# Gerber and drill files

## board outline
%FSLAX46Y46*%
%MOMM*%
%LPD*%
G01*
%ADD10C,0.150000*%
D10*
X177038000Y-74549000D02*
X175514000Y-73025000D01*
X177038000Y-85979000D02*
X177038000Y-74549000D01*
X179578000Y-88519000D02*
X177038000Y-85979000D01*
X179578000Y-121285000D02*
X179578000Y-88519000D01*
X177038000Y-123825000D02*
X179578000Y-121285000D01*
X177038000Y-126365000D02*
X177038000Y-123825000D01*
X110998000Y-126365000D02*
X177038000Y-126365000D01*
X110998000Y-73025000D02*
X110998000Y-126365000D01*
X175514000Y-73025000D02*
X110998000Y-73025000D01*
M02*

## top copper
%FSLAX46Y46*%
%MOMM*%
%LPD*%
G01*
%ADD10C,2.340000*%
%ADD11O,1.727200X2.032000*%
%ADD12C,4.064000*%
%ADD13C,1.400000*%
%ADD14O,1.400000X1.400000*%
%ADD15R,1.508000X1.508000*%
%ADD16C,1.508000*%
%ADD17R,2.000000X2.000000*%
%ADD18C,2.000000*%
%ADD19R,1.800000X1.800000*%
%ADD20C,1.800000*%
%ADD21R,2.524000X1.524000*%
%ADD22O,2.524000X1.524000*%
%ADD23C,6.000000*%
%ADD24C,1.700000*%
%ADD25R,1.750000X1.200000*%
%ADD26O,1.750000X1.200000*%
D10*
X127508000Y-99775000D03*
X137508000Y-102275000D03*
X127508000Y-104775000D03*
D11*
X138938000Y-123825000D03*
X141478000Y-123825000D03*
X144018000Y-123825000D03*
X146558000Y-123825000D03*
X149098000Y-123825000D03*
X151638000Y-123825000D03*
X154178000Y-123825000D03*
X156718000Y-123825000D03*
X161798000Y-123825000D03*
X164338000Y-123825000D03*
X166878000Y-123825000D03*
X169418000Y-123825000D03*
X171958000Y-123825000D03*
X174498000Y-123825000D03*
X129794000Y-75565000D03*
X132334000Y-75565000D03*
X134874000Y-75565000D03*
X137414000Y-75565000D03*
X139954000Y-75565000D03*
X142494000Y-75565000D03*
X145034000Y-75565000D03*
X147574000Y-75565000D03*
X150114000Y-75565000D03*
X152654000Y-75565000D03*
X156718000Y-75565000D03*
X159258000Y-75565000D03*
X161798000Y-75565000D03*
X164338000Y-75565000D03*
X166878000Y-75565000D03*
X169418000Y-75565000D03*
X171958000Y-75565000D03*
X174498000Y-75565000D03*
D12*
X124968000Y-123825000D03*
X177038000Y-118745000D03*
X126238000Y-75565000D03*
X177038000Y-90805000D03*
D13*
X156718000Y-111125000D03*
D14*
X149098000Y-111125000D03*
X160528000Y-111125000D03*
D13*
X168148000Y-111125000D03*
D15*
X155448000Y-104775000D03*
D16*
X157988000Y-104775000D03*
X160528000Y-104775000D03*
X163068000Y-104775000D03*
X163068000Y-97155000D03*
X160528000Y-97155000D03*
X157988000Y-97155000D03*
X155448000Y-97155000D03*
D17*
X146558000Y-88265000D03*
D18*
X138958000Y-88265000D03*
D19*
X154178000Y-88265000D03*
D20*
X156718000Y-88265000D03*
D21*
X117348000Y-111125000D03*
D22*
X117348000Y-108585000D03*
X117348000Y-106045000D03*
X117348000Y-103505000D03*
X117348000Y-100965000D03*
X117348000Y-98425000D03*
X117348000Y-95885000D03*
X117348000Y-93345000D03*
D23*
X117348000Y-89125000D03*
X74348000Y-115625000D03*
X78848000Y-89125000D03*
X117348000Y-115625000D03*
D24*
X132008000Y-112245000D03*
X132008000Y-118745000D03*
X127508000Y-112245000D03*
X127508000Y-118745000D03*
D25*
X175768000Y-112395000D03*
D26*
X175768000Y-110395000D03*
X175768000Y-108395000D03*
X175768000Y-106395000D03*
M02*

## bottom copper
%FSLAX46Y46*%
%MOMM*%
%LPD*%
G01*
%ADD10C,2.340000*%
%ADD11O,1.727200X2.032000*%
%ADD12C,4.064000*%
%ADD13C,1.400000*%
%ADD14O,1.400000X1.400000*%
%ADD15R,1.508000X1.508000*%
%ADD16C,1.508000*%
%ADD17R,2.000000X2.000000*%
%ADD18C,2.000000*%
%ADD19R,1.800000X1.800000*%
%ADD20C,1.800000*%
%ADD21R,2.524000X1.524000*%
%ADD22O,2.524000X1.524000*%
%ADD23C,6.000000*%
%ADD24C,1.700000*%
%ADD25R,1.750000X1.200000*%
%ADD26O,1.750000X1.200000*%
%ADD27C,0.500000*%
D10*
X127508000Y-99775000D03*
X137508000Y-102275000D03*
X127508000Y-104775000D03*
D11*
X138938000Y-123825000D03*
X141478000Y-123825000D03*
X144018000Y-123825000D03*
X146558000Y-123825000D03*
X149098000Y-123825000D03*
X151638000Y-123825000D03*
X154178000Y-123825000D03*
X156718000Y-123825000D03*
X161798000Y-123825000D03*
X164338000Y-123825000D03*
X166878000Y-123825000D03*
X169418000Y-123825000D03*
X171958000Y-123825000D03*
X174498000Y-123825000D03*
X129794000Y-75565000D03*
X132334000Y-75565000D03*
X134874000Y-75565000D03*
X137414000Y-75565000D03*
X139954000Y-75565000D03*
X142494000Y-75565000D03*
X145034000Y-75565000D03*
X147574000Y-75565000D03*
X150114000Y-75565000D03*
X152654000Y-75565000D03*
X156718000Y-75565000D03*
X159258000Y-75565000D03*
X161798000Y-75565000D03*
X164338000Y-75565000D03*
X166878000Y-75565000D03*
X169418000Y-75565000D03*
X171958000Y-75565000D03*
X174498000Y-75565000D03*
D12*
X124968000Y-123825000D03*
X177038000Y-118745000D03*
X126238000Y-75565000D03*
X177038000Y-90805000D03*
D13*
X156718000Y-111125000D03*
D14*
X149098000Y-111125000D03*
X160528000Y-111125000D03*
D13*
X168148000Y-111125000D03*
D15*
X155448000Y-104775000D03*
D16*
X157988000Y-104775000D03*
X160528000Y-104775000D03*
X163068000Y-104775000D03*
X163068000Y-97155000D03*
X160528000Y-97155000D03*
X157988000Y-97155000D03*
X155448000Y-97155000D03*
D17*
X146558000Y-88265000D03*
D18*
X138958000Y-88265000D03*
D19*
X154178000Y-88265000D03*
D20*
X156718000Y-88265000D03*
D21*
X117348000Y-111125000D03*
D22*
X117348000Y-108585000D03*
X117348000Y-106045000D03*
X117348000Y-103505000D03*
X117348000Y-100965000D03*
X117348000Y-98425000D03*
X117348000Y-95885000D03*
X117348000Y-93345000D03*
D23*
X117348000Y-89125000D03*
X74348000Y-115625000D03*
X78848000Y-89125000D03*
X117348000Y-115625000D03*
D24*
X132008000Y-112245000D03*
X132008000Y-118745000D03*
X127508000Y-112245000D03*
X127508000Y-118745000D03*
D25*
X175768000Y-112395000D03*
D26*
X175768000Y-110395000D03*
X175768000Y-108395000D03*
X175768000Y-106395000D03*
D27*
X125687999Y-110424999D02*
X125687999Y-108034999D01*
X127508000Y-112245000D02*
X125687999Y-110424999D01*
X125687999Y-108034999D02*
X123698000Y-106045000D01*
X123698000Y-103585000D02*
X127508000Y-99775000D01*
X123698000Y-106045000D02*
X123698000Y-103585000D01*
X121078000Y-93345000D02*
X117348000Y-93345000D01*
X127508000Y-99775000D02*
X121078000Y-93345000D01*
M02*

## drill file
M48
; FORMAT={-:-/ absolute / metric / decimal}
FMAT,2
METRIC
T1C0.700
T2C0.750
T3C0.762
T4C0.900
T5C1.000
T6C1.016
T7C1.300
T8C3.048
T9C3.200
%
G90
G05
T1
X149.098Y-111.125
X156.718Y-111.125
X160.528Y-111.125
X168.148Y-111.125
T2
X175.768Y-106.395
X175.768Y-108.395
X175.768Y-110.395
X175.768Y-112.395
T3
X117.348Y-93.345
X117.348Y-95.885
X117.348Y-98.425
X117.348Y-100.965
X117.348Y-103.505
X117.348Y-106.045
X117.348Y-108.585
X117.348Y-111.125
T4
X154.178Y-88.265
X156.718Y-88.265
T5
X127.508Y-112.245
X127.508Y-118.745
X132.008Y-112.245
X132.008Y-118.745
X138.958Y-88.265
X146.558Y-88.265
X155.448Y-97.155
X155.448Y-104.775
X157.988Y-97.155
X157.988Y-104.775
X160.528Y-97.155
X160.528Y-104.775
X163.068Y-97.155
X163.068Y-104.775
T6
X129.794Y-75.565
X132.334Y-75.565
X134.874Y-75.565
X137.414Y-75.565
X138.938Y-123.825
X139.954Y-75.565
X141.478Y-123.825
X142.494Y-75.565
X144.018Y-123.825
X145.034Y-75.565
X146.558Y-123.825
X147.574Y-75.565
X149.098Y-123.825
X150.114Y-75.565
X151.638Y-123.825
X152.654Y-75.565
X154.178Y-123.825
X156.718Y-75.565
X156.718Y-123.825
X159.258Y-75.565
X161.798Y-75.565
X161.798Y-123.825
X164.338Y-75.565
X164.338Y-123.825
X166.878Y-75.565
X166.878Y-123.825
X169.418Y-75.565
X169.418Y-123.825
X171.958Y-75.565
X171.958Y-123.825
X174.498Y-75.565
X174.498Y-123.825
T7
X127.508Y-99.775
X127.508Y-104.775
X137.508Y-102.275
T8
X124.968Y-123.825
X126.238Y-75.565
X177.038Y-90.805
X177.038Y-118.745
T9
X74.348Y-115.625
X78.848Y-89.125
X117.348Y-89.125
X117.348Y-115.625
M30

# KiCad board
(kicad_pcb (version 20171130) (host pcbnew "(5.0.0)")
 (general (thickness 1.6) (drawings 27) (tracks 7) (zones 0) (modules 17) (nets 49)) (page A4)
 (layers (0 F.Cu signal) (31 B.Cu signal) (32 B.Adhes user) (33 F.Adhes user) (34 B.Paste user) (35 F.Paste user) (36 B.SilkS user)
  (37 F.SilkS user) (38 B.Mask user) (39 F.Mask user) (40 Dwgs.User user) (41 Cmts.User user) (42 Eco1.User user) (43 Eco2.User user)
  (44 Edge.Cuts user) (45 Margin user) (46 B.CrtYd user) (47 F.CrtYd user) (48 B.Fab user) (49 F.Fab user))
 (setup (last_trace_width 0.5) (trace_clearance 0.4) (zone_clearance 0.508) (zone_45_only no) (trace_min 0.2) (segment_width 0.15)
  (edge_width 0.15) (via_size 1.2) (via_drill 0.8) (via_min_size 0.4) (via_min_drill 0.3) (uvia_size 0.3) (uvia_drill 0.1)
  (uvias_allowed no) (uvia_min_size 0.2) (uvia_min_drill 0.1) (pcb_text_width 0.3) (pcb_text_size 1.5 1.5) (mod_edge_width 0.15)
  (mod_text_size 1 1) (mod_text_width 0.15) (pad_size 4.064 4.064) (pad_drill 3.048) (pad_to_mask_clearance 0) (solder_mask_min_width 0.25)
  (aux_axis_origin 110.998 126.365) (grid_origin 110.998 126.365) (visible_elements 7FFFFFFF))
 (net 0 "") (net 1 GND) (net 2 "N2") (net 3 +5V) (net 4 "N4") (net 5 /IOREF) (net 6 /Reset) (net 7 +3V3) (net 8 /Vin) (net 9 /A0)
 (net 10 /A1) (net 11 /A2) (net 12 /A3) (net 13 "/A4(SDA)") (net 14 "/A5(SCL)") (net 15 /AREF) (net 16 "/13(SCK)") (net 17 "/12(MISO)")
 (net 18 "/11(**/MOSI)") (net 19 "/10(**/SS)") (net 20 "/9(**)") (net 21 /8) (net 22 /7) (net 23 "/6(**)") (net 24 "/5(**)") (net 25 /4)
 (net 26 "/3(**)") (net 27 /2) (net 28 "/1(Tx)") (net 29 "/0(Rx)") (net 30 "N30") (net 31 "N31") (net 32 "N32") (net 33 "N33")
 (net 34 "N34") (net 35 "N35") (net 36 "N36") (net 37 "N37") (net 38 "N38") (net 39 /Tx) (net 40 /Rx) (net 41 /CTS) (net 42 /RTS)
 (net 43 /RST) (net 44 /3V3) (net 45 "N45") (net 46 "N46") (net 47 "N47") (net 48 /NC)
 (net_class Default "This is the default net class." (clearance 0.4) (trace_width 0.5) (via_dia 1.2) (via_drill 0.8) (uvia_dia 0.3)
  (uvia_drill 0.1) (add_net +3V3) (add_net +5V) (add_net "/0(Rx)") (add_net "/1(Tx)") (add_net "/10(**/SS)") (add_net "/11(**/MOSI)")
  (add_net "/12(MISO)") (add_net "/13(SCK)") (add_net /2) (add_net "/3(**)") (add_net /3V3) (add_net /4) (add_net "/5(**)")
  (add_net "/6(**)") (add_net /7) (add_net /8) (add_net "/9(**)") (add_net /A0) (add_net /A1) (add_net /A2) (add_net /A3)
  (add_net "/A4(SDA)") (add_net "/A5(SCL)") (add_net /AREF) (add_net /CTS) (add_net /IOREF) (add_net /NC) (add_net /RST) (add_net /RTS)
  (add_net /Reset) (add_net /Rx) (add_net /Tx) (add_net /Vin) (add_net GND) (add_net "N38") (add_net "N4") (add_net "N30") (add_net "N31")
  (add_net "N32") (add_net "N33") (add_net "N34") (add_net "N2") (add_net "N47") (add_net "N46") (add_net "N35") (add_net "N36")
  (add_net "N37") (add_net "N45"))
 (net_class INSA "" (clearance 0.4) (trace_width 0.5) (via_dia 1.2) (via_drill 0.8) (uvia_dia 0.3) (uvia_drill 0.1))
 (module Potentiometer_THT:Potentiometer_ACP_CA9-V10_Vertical (layer F.Cu) (at 127.508 104.775)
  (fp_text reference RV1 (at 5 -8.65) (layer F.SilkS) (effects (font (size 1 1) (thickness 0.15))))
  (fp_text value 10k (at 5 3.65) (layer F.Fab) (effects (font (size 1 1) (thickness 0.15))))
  (pad 3 thru_hole circle (at 0 -5) (size 2.34 2.34) (drill 1.3) (layers *.Cu *.Mask) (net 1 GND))
  (pad 2 thru_hole circle (at 10 -2.5) (size 2.34 2.34) (drill 1.3) (layers *.Cu *.Mask) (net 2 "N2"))
  (pad 1 thru_hole circle (at 0 0) (size 2.34 2.34) (drill 1.3) (layers *.Cu *.Mask) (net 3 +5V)))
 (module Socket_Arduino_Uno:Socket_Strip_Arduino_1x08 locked (layer F.Cu) (at 138.938 123.825)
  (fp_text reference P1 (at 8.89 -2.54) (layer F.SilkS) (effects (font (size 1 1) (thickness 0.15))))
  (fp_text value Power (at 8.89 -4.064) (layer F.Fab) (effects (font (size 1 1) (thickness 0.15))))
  (pad 1 thru_hole oval (at 0 0) (size 1.7272 2.032) (drill 1.016) (layers *.Cu *.Mask F.SilkS) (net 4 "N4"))
  (pad 2 thru_hole oval (at 2.54 0) (size 1.7272 2.032) (drill 1.016) (layers *.Cu *.Mask F.SilkS) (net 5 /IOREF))
  (pad 3 thru_hole oval (at 5.08 0) (size 1.7272 2.032) (drill 1.016) (layers *.Cu *.Mask F.SilkS) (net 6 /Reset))
  (pad 4 thru_hole oval (at 7.62 0) (size 1.7272 2.032) (drill 1.016) (layers *.Cu *.Mask F.SilkS) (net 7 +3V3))
  (pad 5 thru_hole oval (at 10.16 0) (size 1.7272 2.032) (drill 1.016) (layers *.Cu *.Mask F.SilkS) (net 3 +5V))
  (pad 6 thru_hole oval (at 12.7 0) (size 1.7272 2.032) (drill 1.016) (layers *.Cu *.Mask F.SilkS) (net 1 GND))
  (pad 7 thru_hole oval (at 15.24 0) (size 1.7272 2.032) (drill 1.016) (layers *.Cu *.Mask F.SilkS) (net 1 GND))
  (pad 8 thru_hole oval (at 17.78 0) (size 1.7272 2.032) (drill 1.016) (layers *.Cu *.Mask F.SilkS) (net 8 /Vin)))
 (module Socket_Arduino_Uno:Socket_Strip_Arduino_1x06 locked (layer F.Cu) (at 161.798 123.825)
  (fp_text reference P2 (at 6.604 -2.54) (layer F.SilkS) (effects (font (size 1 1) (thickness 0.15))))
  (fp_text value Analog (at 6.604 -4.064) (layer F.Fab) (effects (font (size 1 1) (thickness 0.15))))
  (pad 1 thru_hole oval (at 0 0) (size 1.7272 2.032) (drill 1.016) (layers *.Cu *.Mask F.SilkS) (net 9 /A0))
  (pad 2 thru_hole oval (at 2.54 0) (size 1.7272 2.032) (drill 1.016) (layers *.Cu *.Mask F.SilkS) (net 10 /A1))
  (pad 3 thru_hole oval (at 5.08 0) (size 1.7272 2.032) (drill 1.016) (layers *.Cu *.Mask F.SilkS) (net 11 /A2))
  (pad 4 thru_hole oval (at 7.62 0) (size 1.7272 2.032) (drill 1.016) (layers *.Cu *.Mask F.SilkS) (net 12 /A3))
  (pad 5 thru_hole oval (at 10.16 0) (size 1.7272 2.032) (drill 1.016) (layers *.Cu *.Mask F.SilkS) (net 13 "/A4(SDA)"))
  (pad 6 thru_hole oval (at 12.7 0) (size 1.7272 2.032) (drill 1.016) (layers *.Cu *.Mask F.SilkS) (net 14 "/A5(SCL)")))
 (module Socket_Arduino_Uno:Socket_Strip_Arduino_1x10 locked (layer F.Cu) (at 129.794 75.565)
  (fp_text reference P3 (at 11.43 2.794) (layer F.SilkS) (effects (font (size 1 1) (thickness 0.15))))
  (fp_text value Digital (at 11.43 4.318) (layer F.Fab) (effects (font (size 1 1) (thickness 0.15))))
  (pad 1 thru_hole oval (at 0 0) (size 1.7272 2.032) (drill 1.016) (layers *.Cu *.Mask F.SilkS) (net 14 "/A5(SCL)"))
  (pad 2 thru_hole oval (at 2.54 0) (size 1.7272 2.032) (drill 1.016) (layers *.Cu *.Mask F.SilkS) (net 13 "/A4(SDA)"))
  (pad 3 thru_hole oval (at 5.08 0) (size 1.7272 2.032) (drill 1.016) (layers *.Cu *.Mask F.SilkS) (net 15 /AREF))
  (pad 4 thru_hole oval (at 7.62 0) (size 1.7272 2.032) (drill 1.016) (layers *.Cu *.Mask F.SilkS) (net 1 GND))
  (pad 5 thru_hole oval (at 10.16 0) (size 1.7272 2.032) (drill 1.016) (layers *.Cu *.Mask F.SilkS) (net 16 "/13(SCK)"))
  (pad 6 thru_hole oval (at 12.7 0) (size 1.7272 2.032) (drill 1.016) (layers *.Cu *.Mask F.SilkS) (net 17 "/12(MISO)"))
  (pad 7 thru_hole oval (at 15.24 0) (size 1.7272 2.032) (drill 1.016) (layers *.Cu *.Mask F.SilkS) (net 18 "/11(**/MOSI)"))
  (pad 8 thru_hole oval (at 17.78 0) (size 1.7272 2.032) (drill 1.016) (layers *.Cu *.Mask F.SilkS) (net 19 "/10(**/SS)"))
  (pad 9 thru_hole oval (at 20.32 0) (size 1.7272 2.032) (drill 1.016) (layers *.Cu *.Mask F.SilkS) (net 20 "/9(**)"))
  (pad 10 thru_hole oval (at 22.86 0) (size 1.7272 2.032) (drill 1.016) (layers *.Cu *.Mask F.SilkS) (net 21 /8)))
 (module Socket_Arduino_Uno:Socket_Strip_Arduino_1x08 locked (layer F.Cu) (at 156.718 75.565)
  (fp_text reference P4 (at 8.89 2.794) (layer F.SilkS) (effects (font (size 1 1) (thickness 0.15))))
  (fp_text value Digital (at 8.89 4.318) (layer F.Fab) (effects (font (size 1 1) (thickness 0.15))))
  (pad 1 thru_hole oval (at 0 0) (size 1.7272 2.032) (drill 1.016) (layers *.Cu *.Mask F.SilkS) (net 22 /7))
  (pad 2 thru_hole oval (at 2.54 0) (size 1.7272 2.032) (drill 1.016) (layers *.Cu *.Mask F.SilkS) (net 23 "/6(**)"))
  (pad 3 thru_hole oval (at 5.08 0) (size 1.7272 2.032) (drill 1.016) (layers *.Cu *.Mask F.SilkS) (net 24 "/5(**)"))
  (pad 4 thru_hole oval (at 7.62 0) (size 1.7272 2.032) (drill 1.016) (layers *.Cu *.Mask F.SilkS) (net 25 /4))
  (pad 5 thru_hole oval (at 10.16 0) (size 1.7272 2.032) (drill 1.016) (layers *.Cu *.Mask F.SilkS) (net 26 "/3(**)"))
  (pad 6 thru_hole oval (at 12.7 0) (size 1.7272 2.032) (drill 1.016) (layers *.Cu *.Mask F.SilkS) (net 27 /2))
  (pad 7 thru_hole oval (at 15.24 0) (size 1.7272 2.032) (drill 1.016) (layers *.Cu *.Mask F.SilkS) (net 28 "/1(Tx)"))
  (pad 8 thru_hole oval (at 17.78 0) (size 1.7272 2.032) (drill 1.016) (layers *.Cu *.Mask F.SilkS) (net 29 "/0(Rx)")))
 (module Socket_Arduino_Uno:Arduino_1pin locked (layer F.Cu) (at 124.968 123.825)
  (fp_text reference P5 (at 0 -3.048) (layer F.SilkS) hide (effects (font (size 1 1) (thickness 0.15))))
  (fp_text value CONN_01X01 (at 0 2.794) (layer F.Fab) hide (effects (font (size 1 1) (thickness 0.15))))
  (pad 1 thru_hole circle (at 0 0) (size 4.064 4.064) (drill 3.048) (layers *.Cu *.Mask F.SilkS) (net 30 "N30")))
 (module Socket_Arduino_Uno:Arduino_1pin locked (layer F.Cu) (at 177.038 118.745)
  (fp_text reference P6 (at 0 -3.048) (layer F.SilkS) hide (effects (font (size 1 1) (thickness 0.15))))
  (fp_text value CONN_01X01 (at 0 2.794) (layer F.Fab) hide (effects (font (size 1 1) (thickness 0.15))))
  (pad 1 thru_hole circle (at 0 0) (size 4.064 4.064) (drill 3.048) (layers *.Cu *.Mask F.SilkS) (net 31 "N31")))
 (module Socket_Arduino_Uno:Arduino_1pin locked (layer F.Cu) (at 126.238 75.565)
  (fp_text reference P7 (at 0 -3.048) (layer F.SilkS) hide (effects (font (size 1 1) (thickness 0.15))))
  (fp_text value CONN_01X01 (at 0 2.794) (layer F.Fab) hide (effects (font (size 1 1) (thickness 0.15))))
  (pad 1 thru_hole circle (at 0 0) (size 4.064 4.064) (drill 3.048) (layers *.Cu *.Mask F.SilkS) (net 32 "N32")))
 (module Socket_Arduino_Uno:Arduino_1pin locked (layer F.Cu) (at 177.038 90.805)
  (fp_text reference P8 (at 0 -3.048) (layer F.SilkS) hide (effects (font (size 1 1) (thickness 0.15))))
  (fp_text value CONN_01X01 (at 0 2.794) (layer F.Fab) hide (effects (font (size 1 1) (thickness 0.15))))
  (pad 1 thru_hole circle (at 0 0) (size 4.064 4.064) (drill 3.048) (layers *.Cu *.Mask F.SilkS) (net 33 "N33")))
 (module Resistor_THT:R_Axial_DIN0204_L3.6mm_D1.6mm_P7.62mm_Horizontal (layer F.Cu) (at 156.718 111.125 180)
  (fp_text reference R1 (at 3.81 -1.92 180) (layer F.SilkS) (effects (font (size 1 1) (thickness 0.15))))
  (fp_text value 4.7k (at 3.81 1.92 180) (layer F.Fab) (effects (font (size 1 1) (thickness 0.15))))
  (pad 1 thru_hole circle (at 0 0 180) (size 1.4 1.4) (drill 0.7) (layers *.Cu *.Mask) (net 9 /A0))
  (pad 2 thru_hole oval (at 7.62 0 180) (size 1.4 1.4) (drill 0.7) (layers *.Cu *.Mask) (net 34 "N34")))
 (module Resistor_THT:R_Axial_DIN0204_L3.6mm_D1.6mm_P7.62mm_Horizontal (layer F.Cu) (at 168.148 111.125 180)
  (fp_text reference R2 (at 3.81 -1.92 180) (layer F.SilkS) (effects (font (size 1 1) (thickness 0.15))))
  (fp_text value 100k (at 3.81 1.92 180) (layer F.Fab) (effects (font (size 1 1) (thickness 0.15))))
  (pad 2 thru_hole oval (at 7.62 0 180) (size 1.4 1.4) (drill 0.7) (layers *.Cu *.Mask) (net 34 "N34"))
  (pad 1 thru_hole circle (at 0 0 180) (size 1.4 1.4) (drill 0.7) (layers *.Cu *.Mask) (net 27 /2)))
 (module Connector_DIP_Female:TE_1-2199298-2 (layer F.Cu) (at 159.258 100.965 90)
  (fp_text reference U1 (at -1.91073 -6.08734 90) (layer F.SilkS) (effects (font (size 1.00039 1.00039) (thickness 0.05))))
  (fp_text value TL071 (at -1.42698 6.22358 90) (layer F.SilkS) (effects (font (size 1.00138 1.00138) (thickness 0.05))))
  (pad 1 thru_hole rect (at -3.81 -3.81 90) (size 1.508 1.508) (drill 1) (layers *.Cu *.Mask) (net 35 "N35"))
  (pad 2 thru_hole circle (at -3.81 -1.27 90) (size 1.508 1.508) (drill 1) (layers *.Cu *.Mask) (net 2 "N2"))
  (pad 3 thru_hole circle (at -3.81 1.27 90) (size 1.508 1.508) (drill 1) (layers *.Cu *.Mask) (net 34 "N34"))
  (pad 4 thru_hole circle (at -3.81 3.81 90) (size 1.508 1.508) (drill 1) (layers *.Cu *.Mask) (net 1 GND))
  (pad 5 thru_hole circle (at 3.81 3.81 90) (size 1.508 1.508) (drill 1) (layers *.Cu *.Mask) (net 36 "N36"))
  (pad 6 thru_hole circle (at 3.81 1.27 90) (size 1.508 1.508) (drill 1) (layers *.Cu *.Mask) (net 27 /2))
  (pad 7 thru_hole circle (at 3.81 -1.27 90) (size 1.508 1.508) (drill 1) (layers *.Cu *.Mask) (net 3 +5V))
  (pad 8 thru_hole circle (at 3.81 -3.81 90) (size 1.508 1.508) (drill 1) (layers *.Cu *.Mask) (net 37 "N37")))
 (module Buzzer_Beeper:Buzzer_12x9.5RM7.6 (layer F.Cu) (at 146.558 88.265 180)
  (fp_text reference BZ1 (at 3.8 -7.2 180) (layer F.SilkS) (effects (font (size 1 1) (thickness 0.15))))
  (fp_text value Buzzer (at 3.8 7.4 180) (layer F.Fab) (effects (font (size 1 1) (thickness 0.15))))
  (pad 1 thru_hole rect (at 0 0 180) (size 2 2) (drill 1) (layers *.Cu *.Mask) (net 20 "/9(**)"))
  (pad 2 thru_hole circle (at 7.6 0 180) (size 2 2) (drill 1) (layers *.Cu *.Mask) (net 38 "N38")))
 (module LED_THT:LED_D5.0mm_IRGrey (layer F.Cu) (at 154.178 88.265)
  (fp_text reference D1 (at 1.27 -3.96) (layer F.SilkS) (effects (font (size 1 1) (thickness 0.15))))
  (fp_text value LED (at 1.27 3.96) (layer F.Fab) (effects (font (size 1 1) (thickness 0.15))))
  (pad 1 thru_hole rect (at 0 0) (size 1.8 1.8) (drill 0.9) (layers *.Cu *.Mask) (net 1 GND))
  (pad 2 thru_hole circle (at 2.54 0) (size 1.8 1.8) (drill 0.9) (layers *.Cu *.Mask) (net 38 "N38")))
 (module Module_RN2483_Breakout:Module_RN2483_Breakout (layer F.Cu) (at 117.348 111.125 90)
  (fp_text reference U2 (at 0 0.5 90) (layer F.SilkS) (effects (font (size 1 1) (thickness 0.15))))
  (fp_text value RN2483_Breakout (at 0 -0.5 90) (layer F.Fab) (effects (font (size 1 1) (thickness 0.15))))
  (pad 1 thru_hole rect (at 0 0 90) (size 1.524 2.524) (drill 0.762) (layers *.Cu *.Mask) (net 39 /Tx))
  (pad 2 thru_hole oval (at 2.54 0 90) (size 1.524 2.524) (drill 0.762) (layers *.Cu *.Mask) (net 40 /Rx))
  (pad 3 thru_hole oval (at 5.08 0 90) (size 1.524 2.524) (drill 0.762) (layers *.Cu *.Mask) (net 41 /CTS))
  (pad 4 thru_hole oval (at 7.62 0 90) (size 1.524 2.524) (drill 0.762) (layers *.Cu *.Mask) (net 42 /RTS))
  (pad 5 thru_hole oval (at 10.16 0 90) (size 1.524 2.524) (drill 0.762) (layers *.Cu *.Mask) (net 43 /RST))
  (pad 6 thru_hole oval (at 12.7 0 90) (size 1.524 2.524) (drill 0.762) (layers *.Cu *.Mask) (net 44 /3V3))
  (pad 7 thru_hole oval (at 15.24 0 90) (size 1.524 2.524) (drill 0.762) (layers *.Cu *.Mask) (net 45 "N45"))
  (pad 8 thru_hole oval (at 17.78 0 90) (size 1.524 2.524) (drill 0.762) (layers *.Cu *.Mask) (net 1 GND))
  (pad "" np_thru_hole circle (at 22 0 90) (size 6 6) (drill 3.2) (layers *.Cu *.Mask))
  (pad "" np_thru_hole circle (at -4.5 -43 90) (size 6 6) (drill 3.2) (layers *.Cu *.Mask))
  (pad "" np_thru_hole circle (at 22 -38.5 90) (size 6 6) (drill 3.2) (layers *.Cu *.Mask))
  (pad "" np_thru_hole circle (at -4.5 0 90) (size 6 6) (drill 3.2) (layers *.Cu *.Mask)))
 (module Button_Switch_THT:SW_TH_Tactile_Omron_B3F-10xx (layer F.Cu) (at 127.508 118.745 90)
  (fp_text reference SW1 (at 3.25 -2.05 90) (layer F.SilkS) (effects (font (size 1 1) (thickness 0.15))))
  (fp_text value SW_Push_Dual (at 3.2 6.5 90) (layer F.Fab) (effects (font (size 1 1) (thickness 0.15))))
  (pad 4 thru_hole circle (at 6.5 4.5 90) (size 1.7 1.7) (drill 1) (layers *.Cu *.Mask) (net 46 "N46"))
  (pad 3 thru_hole circle (at 0 4.5 90) (size 1.7 1.7) (drill 1) (layers *.Cu *.Mask) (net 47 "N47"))
  (pad 2 thru_hole circle (at 6.5 0 90) (size 1.7 1.7) (drill 1) (layers *.Cu *.Mask) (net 1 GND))
  (pad 1 thru_hole circle (at 0 0 90) (size 1.7 1.7) (drill 1) (layers *.Cu *.Mask) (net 6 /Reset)))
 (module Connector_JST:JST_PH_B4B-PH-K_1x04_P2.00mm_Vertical (layer F.Cu) (at 175.768 112.395 90)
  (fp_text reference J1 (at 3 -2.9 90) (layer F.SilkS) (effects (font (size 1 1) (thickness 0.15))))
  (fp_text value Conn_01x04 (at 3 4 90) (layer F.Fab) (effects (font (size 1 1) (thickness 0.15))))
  (pad 1 thru_hole rect (at 0 0 90) (size 1.2 1.75) (drill 0.75) (layers *.Cu *.Mask) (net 1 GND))
  (pad 2 thru_hole oval (at 2 0 90) (size 1.2 1.75) (drill 0.75) (layers *.Cu *.Mask) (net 3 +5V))
  (pad 3 thru_hole oval (at 4 0 90) (size 1.2 1.75) (drill 0.75) (layers *.Cu *.Mask) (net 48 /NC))
  (pad 4 thru_hole oval (at 6 0 90) (size 1.2 1.75) (drill 0.75) (layers *.Cu *.Mask) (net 9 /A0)))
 (gr_line (start 177.038 74.549) (end 175.514 73.025) (angle 90) (layer Edge.Cuts) (width 0.15))
 (gr_line (start 177.038 85.979) (end 177.038 74.549) (angle 90) (layer Edge.Cuts) (width 0.15))
 (gr_line (start 179.578 88.519) (end 177.038 85.979) (angle 90) (layer Edge.Cuts) (width 0.15))
 (gr_line (start 179.578 121.285) (end 179.578 88.519) (angle 90) (layer Edge.Cuts) (width 0.15))
 (gr_line (start 177.038 123.825) (end 179.578 121.285) (angle 90) (layer Edge.Cuts) (width 0.15))
 (gr_line (start 177.038 126.365) (end 177.038 123.825) (angle 90) (layer Edge.Cuts) (width 0.15))
 (gr_line (start 110.998 126.365) (end 177.038 126.365) (angle 90) (layer Edge.Cuts) (width 0.15))
 (gr_line (start 110.998 73.025) (end 110.998 126.365) (angle 90) (layer Edge.Cuts) (width 0.15))
 (gr_line (start 175.514 73.025) (end 110.998 73.025) (angle 90) (layer Edge.Cuts) (width 0.15))
 (segment (start 125.687999 110.424999) (end 125.687999 108.034999) (width 0.5) (layer B.Cu) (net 1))
 (segment (start 127.508 112.245) (end 125.687999 110.424999) (width 0.5) (layer B.Cu) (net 1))
 (segment (start 125.687999 108.034999) (end 123.698 106.045) (width 0.5) (layer B.Cu) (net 1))
 (segment (start 123.698 103.585) (end 127.508 99.775) (width 0.5) (layer B.Cu) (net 1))
 (segment (start 123.698 106.045) (end 123.698 103.585) (width 0.5) (layer B.Cu) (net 1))
 (segment (start 121.078 93.345) (end 117.348 93.345) (width 0.5) (layer B.Cu) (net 1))
 (segment (start 127.508 99.775) (end 121.078 93.345) (width 0.5) (layer B.Cu) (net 1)))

